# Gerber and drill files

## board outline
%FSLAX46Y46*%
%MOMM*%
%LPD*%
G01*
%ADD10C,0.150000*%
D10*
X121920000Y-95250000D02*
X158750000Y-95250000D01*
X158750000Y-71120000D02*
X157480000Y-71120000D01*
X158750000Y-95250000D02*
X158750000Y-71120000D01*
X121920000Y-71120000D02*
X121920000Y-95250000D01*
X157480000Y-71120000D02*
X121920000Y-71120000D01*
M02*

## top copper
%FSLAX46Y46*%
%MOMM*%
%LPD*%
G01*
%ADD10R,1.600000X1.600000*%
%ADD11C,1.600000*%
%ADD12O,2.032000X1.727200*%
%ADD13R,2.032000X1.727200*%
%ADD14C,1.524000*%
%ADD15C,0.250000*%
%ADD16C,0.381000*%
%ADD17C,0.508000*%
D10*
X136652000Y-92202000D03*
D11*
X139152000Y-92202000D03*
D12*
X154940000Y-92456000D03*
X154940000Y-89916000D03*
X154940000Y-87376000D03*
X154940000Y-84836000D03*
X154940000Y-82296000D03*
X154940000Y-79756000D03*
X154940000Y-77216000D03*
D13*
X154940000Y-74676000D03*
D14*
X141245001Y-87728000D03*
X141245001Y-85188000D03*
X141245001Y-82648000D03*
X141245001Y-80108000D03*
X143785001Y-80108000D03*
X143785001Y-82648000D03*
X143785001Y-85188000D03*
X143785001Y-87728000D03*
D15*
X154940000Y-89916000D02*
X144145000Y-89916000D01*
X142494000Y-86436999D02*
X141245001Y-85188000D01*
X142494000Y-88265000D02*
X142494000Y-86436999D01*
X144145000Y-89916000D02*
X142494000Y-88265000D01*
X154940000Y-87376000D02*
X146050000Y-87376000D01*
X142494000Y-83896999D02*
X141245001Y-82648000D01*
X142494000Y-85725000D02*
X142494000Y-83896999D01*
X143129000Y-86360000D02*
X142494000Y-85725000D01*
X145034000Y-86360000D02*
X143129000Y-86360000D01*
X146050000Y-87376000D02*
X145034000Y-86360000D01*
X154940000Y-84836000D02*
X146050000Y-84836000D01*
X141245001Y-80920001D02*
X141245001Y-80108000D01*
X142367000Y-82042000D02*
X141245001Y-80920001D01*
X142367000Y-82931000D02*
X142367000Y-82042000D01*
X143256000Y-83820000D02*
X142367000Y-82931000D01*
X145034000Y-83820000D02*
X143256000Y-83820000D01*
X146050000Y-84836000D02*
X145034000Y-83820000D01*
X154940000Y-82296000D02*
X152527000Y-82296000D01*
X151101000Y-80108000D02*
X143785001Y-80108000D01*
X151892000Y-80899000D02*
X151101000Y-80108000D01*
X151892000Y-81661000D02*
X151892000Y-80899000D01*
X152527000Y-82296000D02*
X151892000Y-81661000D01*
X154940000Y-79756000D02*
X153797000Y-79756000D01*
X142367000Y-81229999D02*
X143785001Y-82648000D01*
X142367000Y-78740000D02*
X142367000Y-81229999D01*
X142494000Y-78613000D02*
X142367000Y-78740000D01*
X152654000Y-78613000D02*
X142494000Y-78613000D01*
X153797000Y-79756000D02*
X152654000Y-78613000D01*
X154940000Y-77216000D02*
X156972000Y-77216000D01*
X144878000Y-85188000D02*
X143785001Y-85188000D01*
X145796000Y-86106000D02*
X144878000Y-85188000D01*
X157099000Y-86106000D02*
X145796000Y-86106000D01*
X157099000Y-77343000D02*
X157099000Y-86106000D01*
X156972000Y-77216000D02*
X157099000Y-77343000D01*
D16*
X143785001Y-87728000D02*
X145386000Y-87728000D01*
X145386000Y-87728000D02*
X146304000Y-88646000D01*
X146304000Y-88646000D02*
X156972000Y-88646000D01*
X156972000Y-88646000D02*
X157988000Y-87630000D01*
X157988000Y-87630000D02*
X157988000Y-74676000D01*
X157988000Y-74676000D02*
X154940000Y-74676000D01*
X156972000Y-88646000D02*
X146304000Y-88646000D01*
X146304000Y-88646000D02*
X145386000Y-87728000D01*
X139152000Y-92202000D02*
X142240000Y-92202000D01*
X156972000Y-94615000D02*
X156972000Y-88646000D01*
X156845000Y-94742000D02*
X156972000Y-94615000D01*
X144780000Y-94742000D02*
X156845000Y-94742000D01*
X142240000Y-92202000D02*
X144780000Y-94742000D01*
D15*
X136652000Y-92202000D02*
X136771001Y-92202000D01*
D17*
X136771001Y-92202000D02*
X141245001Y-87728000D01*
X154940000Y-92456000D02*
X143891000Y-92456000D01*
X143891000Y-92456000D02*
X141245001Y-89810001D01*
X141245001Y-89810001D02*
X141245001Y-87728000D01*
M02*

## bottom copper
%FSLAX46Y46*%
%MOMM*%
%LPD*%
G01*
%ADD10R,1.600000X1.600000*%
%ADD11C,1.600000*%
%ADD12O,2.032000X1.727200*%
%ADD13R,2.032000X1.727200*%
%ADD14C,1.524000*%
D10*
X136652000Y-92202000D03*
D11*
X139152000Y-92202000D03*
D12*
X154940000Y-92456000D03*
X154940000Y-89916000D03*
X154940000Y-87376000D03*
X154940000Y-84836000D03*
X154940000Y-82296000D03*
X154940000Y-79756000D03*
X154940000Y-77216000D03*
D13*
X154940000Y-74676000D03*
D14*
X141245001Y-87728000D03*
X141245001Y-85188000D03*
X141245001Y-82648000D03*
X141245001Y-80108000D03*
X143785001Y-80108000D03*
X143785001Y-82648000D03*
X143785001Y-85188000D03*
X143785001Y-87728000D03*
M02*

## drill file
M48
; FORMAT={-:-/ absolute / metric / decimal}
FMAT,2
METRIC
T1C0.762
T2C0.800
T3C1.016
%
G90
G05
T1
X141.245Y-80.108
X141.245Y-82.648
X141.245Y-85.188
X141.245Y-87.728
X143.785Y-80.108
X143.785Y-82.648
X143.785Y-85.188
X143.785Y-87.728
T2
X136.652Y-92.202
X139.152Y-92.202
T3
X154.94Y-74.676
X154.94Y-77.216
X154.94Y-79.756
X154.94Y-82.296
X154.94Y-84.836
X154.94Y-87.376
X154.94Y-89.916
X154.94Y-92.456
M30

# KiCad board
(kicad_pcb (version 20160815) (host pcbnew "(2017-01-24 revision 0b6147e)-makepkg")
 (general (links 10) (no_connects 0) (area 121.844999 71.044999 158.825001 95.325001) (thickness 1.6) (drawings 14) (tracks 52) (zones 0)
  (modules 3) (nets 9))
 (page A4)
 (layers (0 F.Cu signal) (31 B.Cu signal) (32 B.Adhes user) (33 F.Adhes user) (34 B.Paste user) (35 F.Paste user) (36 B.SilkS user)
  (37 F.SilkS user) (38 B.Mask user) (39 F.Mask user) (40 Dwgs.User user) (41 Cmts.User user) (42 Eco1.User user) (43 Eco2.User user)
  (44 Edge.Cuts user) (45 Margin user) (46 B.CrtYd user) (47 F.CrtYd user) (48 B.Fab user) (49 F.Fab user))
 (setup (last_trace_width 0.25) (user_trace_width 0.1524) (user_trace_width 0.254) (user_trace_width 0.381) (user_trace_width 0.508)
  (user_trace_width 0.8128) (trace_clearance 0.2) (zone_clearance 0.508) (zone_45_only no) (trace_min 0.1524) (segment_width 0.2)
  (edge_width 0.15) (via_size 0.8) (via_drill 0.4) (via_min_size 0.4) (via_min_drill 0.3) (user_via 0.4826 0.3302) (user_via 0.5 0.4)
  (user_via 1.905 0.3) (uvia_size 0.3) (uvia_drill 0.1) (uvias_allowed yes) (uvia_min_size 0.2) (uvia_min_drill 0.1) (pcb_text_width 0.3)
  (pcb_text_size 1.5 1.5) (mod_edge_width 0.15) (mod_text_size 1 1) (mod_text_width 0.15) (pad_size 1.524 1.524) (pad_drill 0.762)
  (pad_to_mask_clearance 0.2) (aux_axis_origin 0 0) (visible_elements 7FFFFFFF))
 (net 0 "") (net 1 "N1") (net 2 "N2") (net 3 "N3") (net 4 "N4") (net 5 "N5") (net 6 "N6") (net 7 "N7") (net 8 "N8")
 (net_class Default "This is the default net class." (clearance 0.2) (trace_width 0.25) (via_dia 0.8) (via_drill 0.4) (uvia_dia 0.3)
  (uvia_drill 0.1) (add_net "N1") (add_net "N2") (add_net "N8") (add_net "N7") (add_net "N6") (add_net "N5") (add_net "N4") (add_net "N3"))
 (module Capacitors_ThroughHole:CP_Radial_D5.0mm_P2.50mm (layer F.Cu) (at 136.652 92.202)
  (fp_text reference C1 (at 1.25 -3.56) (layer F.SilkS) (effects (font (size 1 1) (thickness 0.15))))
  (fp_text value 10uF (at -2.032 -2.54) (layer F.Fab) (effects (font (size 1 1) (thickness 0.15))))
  (pad 1 thru_hole rect (at 0 0) (size 1.6 1.6) (drill 0.8) (layers *.Cu *.Mask) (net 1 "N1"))
  (pad 2 thru_hole circle (at 2.5 0) (size 1.6 1.6) (drill 0.8) (layers *.Cu *.Mask) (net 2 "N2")))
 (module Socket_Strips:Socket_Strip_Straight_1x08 (layer F.Cu) (at 154.94 74.676 270)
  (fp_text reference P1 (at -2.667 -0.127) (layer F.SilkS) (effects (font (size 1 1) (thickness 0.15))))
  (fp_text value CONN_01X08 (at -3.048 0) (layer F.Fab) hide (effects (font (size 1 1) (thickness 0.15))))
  (pad 8 thru_hole oval (at 17.78 0 270) (size 1.7272 2.032) (drill 1.016) (layers *.Cu *.Mask) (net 1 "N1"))
  (pad 7 thru_hole oval (at 15.24 0 270) (size 1.7272 2.032) (drill 1.016) (layers *.Cu *.Mask) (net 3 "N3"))
  (pad 6 thru_hole oval (at 12.7 0 270) (size 1.7272 2.032) (drill 1.016) (layers *.Cu *.Mask) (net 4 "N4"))
  (pad 5 thru_hole oval (at 10.16 0 270) (size 1.7272 2.032) (drill 1.016) (layers *.Cu *.Mask) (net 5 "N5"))
  (pad 4 thru_hole oval (at 7.62 0 270) (size 1.7272 2.032) (drill 1.016) (layers *.Cu *.Mask) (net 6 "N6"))
  (pad 3 thru_hole oval (at 5.08 0 270) (size 1.7272 2.032) (drill 1.016) (layers *.Cu *.Mask) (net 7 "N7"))
  (pad 2 thru_hole oval (at 2.54 0 270) (size 1.7272 2.032) (drill 1.016) (layers *.Cu *.Mask) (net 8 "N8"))
  (pad 1 thru_hole rect (at 0 0 270) (size 1.7272 2.032) (drill 1.016) (layers *.Cu *.Mask) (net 2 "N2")))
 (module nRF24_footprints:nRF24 (layer F.Cu) (at 133.625001 77.568)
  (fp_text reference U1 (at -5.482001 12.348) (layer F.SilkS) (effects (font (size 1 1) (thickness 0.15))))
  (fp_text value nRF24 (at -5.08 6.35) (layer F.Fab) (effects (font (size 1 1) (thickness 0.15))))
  (pad 7 thru_hole circle (at 7.62 10.16) (size 1.524 1.524) (drill 0.762) (layers *.Cu *.Mask) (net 1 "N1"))
  (pad 6 thru_hole circle (at 7.62 7.62) (size 1.524 1.524) (drill 0.762) (layers *.Cu *.Mask) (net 3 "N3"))
  (pad 5 thru_hole circle (at 7.62 5.08) (size 1.524 1.524) (drill 0.762) (layers *.Cu *.Mask) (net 4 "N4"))
  (pad 4 thru_hole circle (at 7.62 2.54) (size 1.524 1.524) (drill 0.762) (layers *.Cu *.Mask) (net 5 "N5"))
  (pad 3 thru_hole circle (at 10.16 2.54) (size 1.524 1.524) (drill 0.762) (layers *.Cu *.Mask) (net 6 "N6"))
  (pad 2 thru_hole circle (at 10.16 5.08) (size 1.524 1.524) (drill 0.762) (layers *.Cu *.Mask) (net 7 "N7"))
  (pad 1 thru_hole circle (at 10.16 7.62) (size 1.524 1.524) (drill 0.762) (layers *.Cu *.Mask) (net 8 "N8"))
  (pad 0 thru_hole circle (at 10.16 10.16) (size 1.524 1.524) (drill 0.762) (layers *.Cu *.Mask) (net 2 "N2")))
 (gr_line (start 121.92 95.25) (end 158.75 95.25) (angle 90) (layer Edge.Cuts) (width 0.15))
 (gr_line (start 158.75 71.12) (end 157.48 71.12) (angle 90) (layer Edge.Cuts) (width 0.15))
 (gr_line (start 158.75 95.25) (end 158.75 71.12) (angle 90) (layer Edge.Cuts) (width 0.15))
 (gr_line (start 121.92 71.12) (end 121.92 95.25) (angle 90) (layer Edge.Cuts) (width 0.15))
 (gr_line (start 157.48 71.12) (end 121.92 71.12) (angle 90) (layer Edge.Cuts) (width 0.15))
 (segment (start 154.94 89.916) (end 144.145 89.916) (width 0.25) (layer F.Cu) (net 3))
 (segment (start 142.494 86.436999) (end 141.245001 85.188) (width 0.25) (layer F.Cu) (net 3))
 (segment (start 142.494 88.265) (end 142.494 86.436999) (width 0.25) (layer F.Cu) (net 3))
 (segment (start 144.145 89.916) (end 142.494 88.265) (width 0.25) (layer F.Cu) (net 3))
 (segment (start 154.94 87.376) (end 146.05 87.376) (width 0.25) (layer F.Cu) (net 4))
 (segment (start 142.494 83.896999) (end 141.245001 82.648) (width 0.25) (layer F.Cu) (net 4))
 (segment (start 142.494 85.725) (end 142.494 83.896999) (width 0.25) (layer F.Cu) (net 4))
 (segment (start 143.129 86.36) (end 142.494 85.725) (width 0.25) (layer F.Cu) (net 4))
 (segment (start 145.034 86.36) (end 143.129 86.36) (width 0.25) (layer F.Cu) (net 4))
 (segment (start 146.05 87.376) (end 145.034 86.36) (width 0.25) (layer F.Cu) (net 4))
 (segment (start 154.94 84.836) (end 146.05 84.836) (width 0.25) (layer F.Cu) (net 5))
 (segment (start 141.245001 80.920001) (end 141.245001 80.108) (width 0.25) (layer F.Cu) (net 5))
 (segment (start 142.367 82.042) (end 141.245001 80.920001) (width 0.25) (layer F.Cu) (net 5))
 (segment (start 142.367 82.931) (end 142.367 82.042) (width 0.25) (layer F.Cu) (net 5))
 (segment (start 143.256 83.82) (end 142.367 82.931) (width 0.25) (layer F.Cu) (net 5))
 (segment (start 145.034 83.82) (end 143.256 83.82) (width 0.25) (layer F.Cu) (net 5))
 (segment (start 146.05 84.836) (end 145.034 83.82) (width 0.25) (layer F.Cu) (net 5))
 (segment (start 154.94 82.296) (end 152.527 82.296) (width 0.25) (layer F.Cu) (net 6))
 (segment (start 151.101 80.108) (end 143.785001 80.108) (width 0.25) (layer F.Cu) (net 6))
 (segment (start 151.892 80.899) (end 151.101 80.108) (width 0.25) (layer F.Cu) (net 6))
 (segment (start 151.892 81.661) (end 151.892 80.899) (width 0.25) (layer F.Cu) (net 6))
 (segment (start 152.527 82.296) (end 151.892 81.661) (width 0.25) (layer F.Cu) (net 6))
 (segment (start 154.94 79.756) (end 153.797 79.756) (width 0.25) (layer F.Cu) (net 7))
 (segment (start 142.367 81.229999) (end 143.785001 82.648) (width 0.25) (layer F.Cu) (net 7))
 (segment (start 142.367 78.74) (end 142.367 81.229999) (width 0.25) (layer F.Cu) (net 7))
 (segment (start 142.494 78.613) (end 142.367 78.74) (width 0.25) (layer F.Cu) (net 7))
 (segment (start 152.654 78.613) (end 142.494 78.613) (width 0.25) (layer F.Cu) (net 7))
 (segment (start 153.797 79.756) (end 152.654 78.613) (width 0.25) (layer F.Cu) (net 7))
 (segment (start 154.94 77.216) (end 156.972 77.216) (width 0.25) (layer F.Cu) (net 8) (status 400000))
 (segment (start 144.878 85.188) (end 143.785001 85.188) (width 0.25) (layer F.Cu) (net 8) (status 800000))
 (segment (start 145.796 86.106) (end 144.878 85.188) (width 0.25) (layer F.Cu) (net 8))
 (segment (start 157.099 86.106) (end 145.796 86.106) (width 0.25) (layer F.Cu) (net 8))
 (segment (start 157.099 77.343) (end 157.099 86.106) (width 0.25) (layer F.Cu) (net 8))
 (segment (start 156.972 77.216) (end 157.099 77.343) (width 0.25) (layer F.Cu) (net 8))
 (segment (start 143.785001 87.728) (end 145.386 87.728) (width 0.381) (layer F.Cu) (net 2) (status 400000))
 (segment (start 145.386 87.728) (end 146.304 88.646) (width 0.381) (layer F.Cu) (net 2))
 (segment (start 146.304 88.646) (end 156.972 88.646) (width 0.381) (layer F.Cu) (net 2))
 (segment (start 156.972 88.646) (end 157.988 87.63) (width 0.381) (layer F.Cu) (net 2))
 (segment (start 157.988 87.63) (end 157.988 74.676) (width 0.381) (layer F.Cu) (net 2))
 (segment (start 157.988 74.676) (end 154.94 74.676) (width 0.381) (layer F.Cu) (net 2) (status 800000))
 (segment (start 156.972 88.646) (end 146.304 88.646) (width 0.381) (layer F.Cu) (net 2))
 (segment (start 146.304 88.646) (end 145.386 87.728) (width 0.381) (layer F.Cu) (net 2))
 (segment (start 139.152 92.202) (end 142.24 92.202) (width 0.381) (layer F.Cu) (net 2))
 (segment (start 156.972 94.615) (end 156.972 88.646) (width 0.381) (layer F.Cu) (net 2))
 (segment (start 156.845 94.742) (end 156.972 94.615) (width 0.381) (layer F.Cu) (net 2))
 (segment (start 144.78 94.742) (end 156.845 94.742) (width 0.381) (layer F.Cu) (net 2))
 (segment (start 142.24 92.202) (end 144.78 94.742) (width 0.381) (layer F.Cu) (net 2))
 (segment (start 136.652 92.202) (end 136.771001 92.202) (width 0.25) (layer F.Cu) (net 1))
 (segment (start 136.771001 92.202) (end 141.245001 87.728) (width 0.508) (layer F.Cu) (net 1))
 (segment (start 154.94 92.456) (end 143.891 92.456) (width 0.508) (layer F.Cu) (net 1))
 (segment (start 143.891 92.456) (end 141.245001 89.810001) (width 0.508) (layer F.Cu) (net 1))
 (segment (start 141.245001 89.810001) (end 141.245001 87.728) (width 0.508) (layer F.Cu) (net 1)))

